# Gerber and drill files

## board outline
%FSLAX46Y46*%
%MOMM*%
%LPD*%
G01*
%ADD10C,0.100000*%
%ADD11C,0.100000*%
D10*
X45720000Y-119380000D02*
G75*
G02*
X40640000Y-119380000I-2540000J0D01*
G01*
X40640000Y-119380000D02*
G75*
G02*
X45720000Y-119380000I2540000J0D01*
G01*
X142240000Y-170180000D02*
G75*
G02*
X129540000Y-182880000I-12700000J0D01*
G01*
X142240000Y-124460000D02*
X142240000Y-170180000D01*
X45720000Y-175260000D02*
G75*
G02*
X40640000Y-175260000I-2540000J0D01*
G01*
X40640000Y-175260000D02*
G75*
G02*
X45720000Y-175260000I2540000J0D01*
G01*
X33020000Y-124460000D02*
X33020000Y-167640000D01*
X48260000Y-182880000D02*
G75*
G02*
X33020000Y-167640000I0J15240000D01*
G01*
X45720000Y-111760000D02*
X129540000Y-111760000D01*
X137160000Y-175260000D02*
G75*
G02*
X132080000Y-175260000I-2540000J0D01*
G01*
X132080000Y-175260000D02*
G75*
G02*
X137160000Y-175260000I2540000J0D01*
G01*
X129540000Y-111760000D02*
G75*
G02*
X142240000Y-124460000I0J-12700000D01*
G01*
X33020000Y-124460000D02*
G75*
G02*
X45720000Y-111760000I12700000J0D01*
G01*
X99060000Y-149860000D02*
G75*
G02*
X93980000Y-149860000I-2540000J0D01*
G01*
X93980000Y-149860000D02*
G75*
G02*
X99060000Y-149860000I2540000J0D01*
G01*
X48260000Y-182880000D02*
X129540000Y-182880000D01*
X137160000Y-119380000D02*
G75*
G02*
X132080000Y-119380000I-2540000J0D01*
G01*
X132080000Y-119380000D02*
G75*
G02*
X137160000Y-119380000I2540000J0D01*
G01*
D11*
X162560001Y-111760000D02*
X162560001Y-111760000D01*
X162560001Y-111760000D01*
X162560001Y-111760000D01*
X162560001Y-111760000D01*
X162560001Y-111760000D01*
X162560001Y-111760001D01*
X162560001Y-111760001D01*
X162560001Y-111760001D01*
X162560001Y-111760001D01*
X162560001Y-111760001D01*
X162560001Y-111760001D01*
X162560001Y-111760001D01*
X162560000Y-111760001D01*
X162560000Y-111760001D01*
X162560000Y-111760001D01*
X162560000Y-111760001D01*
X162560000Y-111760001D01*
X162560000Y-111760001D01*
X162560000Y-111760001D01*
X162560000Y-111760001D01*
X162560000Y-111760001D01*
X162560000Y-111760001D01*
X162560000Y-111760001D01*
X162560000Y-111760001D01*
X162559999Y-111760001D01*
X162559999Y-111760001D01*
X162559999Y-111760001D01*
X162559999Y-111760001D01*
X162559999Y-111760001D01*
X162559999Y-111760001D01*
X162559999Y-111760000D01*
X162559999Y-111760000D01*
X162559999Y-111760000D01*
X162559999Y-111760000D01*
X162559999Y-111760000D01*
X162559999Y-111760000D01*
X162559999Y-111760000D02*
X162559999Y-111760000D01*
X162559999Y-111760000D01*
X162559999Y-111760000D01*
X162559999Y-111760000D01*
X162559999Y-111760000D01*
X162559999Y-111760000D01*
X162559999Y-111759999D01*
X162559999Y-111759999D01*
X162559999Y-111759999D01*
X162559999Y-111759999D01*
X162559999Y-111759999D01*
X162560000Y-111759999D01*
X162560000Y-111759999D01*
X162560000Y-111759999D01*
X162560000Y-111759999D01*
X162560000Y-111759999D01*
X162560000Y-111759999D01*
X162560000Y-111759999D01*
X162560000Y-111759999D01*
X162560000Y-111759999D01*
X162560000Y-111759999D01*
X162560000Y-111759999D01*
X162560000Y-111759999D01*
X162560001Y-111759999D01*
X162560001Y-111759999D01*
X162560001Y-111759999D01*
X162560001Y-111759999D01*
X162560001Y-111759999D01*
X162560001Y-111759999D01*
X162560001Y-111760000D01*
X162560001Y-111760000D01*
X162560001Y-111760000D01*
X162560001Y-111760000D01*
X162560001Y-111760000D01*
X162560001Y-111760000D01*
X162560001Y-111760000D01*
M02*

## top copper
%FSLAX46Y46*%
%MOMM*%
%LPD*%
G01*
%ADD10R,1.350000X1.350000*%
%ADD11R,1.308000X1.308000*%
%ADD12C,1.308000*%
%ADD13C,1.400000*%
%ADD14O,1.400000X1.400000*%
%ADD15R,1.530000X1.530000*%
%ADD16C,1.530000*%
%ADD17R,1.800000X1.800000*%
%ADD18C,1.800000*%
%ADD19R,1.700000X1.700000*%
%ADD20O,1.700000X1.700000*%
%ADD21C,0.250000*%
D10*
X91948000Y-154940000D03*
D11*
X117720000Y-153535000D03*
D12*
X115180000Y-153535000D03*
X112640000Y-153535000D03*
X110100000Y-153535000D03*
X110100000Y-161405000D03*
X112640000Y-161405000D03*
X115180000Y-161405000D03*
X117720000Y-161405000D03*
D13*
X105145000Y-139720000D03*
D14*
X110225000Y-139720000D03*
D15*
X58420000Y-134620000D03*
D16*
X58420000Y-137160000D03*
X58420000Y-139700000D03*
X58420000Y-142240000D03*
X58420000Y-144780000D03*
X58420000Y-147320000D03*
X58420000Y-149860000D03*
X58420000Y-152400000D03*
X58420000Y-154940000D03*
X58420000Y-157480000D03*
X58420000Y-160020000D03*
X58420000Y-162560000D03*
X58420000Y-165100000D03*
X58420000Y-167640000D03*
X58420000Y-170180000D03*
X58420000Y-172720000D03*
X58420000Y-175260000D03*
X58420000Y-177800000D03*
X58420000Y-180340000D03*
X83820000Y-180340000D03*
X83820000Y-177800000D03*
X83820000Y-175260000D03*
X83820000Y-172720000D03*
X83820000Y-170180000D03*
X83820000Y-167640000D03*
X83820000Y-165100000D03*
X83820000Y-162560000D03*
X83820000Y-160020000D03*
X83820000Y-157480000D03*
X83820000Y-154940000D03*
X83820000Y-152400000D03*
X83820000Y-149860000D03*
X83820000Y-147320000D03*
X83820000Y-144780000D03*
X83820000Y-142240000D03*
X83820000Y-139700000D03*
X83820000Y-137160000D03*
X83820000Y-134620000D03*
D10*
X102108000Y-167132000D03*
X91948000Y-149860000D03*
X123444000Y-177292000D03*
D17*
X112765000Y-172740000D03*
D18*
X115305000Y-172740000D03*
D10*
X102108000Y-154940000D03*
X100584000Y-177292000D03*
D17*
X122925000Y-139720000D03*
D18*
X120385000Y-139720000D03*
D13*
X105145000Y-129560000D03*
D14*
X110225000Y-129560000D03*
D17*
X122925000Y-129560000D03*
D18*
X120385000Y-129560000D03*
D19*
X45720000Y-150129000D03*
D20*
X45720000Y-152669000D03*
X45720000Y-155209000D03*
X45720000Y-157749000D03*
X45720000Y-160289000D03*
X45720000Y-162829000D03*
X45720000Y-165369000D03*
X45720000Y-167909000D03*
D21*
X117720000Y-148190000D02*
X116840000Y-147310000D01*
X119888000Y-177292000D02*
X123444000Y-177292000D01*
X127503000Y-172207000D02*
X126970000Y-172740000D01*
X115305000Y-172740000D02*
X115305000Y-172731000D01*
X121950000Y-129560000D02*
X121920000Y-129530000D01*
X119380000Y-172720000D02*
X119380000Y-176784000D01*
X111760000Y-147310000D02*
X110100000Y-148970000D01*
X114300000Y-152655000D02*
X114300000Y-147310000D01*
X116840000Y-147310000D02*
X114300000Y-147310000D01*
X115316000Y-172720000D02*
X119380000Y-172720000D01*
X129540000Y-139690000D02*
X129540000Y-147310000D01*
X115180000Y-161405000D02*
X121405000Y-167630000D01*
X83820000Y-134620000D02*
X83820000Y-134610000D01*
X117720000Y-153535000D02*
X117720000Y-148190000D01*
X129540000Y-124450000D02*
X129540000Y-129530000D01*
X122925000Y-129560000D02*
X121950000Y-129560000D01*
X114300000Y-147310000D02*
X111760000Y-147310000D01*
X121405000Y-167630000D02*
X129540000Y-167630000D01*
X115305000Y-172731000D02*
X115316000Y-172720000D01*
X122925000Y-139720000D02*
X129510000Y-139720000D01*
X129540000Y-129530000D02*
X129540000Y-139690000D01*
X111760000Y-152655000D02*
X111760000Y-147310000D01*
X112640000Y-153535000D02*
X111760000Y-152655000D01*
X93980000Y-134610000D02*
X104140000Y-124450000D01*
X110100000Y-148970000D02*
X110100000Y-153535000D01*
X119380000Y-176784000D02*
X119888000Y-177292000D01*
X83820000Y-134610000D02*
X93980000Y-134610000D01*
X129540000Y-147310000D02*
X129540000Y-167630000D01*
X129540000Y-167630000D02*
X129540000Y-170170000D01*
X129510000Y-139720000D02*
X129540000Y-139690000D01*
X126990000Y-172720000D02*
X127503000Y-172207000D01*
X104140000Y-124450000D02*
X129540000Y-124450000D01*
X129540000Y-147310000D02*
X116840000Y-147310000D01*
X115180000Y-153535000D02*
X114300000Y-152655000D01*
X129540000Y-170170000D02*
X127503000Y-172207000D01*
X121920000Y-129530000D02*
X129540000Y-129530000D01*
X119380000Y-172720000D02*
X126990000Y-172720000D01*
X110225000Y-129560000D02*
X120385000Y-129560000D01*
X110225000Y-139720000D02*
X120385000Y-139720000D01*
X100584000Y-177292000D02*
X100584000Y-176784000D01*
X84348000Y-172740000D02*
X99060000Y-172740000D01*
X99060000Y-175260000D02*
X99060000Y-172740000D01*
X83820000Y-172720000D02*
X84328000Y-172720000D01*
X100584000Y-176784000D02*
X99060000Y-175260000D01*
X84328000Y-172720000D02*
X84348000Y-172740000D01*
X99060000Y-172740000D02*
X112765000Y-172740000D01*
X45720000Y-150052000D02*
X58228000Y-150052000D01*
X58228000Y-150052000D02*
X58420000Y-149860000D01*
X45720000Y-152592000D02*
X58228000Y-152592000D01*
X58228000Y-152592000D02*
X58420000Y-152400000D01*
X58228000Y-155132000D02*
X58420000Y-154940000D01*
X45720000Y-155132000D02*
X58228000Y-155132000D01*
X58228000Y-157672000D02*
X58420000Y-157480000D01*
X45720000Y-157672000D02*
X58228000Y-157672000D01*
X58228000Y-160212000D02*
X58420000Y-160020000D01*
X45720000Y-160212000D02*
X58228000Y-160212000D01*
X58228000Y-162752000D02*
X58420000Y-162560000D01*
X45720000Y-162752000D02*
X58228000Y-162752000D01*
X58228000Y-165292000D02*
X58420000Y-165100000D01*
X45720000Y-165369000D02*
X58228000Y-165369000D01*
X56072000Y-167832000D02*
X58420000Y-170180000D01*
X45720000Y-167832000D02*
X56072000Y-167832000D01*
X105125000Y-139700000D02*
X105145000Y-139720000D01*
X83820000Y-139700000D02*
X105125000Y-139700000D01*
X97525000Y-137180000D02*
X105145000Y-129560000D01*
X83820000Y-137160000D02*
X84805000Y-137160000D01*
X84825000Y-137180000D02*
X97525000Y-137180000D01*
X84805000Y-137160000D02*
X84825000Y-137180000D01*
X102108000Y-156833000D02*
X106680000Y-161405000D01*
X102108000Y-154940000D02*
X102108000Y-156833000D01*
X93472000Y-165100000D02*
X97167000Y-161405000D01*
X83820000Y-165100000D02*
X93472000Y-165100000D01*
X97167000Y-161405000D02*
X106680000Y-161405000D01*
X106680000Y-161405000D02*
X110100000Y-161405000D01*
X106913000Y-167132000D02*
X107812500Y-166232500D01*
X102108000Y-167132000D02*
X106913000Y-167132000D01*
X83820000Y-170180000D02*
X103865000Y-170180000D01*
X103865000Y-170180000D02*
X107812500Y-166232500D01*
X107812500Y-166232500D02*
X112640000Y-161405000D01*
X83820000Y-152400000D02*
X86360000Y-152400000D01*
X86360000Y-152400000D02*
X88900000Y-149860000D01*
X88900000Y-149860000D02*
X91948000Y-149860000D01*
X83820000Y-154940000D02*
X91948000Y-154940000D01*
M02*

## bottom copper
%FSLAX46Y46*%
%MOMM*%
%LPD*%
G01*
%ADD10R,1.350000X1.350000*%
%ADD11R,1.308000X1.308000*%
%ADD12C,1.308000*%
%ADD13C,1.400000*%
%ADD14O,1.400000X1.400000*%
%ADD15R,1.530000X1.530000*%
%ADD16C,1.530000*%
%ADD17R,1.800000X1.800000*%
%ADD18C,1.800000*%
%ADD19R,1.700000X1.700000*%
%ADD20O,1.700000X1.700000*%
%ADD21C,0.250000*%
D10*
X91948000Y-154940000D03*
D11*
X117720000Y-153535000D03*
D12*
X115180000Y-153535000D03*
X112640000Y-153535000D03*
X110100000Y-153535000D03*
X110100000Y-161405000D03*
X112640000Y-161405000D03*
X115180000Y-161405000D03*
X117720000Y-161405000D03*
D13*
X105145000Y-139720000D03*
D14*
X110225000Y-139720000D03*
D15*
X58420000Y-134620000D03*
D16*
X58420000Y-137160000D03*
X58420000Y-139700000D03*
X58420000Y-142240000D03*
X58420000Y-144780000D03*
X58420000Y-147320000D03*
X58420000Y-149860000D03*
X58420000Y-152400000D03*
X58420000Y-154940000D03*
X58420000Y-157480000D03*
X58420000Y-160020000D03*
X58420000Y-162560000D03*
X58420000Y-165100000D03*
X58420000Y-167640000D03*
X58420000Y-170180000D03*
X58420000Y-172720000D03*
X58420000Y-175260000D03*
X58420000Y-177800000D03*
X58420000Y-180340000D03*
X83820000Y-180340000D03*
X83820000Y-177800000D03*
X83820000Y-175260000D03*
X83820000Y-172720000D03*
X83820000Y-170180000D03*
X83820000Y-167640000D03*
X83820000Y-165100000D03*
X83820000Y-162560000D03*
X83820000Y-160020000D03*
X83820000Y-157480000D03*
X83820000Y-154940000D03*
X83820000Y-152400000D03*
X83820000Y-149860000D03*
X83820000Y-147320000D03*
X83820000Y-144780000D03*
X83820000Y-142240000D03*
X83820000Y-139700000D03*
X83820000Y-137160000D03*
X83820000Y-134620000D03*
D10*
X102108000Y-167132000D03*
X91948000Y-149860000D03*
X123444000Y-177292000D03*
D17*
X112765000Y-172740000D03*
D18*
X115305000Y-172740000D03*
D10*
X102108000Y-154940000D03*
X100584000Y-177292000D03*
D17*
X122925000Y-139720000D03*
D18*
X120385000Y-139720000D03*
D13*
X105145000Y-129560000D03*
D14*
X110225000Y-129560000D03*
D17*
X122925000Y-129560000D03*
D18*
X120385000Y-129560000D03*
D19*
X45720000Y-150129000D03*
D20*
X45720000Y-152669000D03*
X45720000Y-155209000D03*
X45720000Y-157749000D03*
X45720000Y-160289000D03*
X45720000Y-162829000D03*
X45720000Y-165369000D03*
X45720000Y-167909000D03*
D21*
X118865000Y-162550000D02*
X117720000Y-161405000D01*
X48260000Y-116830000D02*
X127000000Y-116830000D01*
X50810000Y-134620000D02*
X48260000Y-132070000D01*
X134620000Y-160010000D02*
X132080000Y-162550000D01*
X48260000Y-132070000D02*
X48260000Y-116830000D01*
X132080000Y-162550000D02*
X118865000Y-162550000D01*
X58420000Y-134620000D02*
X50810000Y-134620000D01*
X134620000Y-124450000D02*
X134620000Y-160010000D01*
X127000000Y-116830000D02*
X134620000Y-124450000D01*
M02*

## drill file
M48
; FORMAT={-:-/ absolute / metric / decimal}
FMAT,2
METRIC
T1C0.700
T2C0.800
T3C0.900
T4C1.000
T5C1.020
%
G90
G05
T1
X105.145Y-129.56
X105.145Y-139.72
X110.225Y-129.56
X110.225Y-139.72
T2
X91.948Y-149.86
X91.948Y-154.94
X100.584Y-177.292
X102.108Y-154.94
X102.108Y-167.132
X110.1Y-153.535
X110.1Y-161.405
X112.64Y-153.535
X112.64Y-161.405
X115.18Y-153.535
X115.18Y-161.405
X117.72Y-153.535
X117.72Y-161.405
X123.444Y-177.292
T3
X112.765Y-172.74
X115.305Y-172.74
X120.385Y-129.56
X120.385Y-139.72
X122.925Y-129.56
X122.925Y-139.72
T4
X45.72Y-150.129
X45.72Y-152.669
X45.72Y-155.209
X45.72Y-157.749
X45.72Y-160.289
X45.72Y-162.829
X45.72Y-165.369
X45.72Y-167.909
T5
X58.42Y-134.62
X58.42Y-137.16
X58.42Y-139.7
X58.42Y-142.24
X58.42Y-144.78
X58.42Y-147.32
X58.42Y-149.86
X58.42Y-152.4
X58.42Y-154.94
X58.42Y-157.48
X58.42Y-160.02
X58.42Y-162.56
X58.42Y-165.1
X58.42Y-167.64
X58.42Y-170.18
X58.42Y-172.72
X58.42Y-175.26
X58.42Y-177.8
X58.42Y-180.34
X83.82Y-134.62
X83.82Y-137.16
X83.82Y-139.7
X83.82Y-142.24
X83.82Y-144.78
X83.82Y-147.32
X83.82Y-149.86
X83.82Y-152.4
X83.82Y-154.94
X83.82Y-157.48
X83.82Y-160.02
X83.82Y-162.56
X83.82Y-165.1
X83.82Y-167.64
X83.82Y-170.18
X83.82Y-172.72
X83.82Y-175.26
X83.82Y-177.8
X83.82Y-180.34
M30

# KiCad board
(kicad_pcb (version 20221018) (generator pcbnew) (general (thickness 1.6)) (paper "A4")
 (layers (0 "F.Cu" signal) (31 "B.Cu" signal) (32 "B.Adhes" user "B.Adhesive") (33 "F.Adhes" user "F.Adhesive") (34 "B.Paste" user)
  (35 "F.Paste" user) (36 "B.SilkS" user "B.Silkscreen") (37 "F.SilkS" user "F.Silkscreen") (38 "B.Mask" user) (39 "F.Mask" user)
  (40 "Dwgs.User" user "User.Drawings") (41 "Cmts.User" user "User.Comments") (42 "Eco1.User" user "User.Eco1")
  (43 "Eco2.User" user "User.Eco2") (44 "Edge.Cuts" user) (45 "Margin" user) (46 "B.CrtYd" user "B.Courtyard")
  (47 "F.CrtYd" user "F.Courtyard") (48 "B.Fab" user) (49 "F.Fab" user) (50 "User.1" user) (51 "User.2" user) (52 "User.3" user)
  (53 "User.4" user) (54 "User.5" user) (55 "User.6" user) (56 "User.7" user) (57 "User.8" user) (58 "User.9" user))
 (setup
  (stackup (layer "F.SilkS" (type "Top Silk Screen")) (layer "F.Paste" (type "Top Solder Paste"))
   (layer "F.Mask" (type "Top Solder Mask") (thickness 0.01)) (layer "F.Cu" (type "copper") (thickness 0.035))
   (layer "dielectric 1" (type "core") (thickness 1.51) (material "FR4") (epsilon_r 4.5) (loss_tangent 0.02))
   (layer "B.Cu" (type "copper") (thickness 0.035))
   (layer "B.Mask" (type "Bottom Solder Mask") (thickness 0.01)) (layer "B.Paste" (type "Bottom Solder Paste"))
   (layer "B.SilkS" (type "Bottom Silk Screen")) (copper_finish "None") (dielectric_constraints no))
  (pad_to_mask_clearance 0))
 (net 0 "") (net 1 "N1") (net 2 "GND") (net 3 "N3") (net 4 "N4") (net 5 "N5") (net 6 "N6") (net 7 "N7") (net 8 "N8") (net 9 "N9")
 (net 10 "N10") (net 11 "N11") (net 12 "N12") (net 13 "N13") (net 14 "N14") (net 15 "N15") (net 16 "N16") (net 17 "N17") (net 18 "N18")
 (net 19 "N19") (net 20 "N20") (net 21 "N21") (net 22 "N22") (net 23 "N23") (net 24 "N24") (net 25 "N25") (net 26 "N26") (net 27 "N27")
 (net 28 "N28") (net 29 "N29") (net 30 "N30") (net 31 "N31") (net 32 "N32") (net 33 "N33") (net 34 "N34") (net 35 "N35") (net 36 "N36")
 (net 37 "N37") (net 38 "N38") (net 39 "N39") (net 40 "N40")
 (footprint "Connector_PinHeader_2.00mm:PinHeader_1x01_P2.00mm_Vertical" (layer "F.Cu") (at 91.948 154.94)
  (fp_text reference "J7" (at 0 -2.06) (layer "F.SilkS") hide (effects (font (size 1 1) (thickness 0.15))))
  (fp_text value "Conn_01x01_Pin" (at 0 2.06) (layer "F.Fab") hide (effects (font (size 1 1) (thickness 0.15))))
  (pad "1" thru_hole rect (at 0 0) (size 1.35 1.35) (drill 0.8) (layers "*.Cu" "*.Mask") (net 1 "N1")))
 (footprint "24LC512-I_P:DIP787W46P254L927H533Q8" (layer "F.Cu") (at 113.91 157.47 -90)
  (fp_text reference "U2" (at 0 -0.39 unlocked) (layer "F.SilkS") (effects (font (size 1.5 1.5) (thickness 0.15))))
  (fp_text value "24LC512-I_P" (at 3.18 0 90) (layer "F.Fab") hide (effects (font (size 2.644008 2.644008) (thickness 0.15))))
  (pad "1" thru_hole rect (at -3.935 -3.81 270) (size 1.308 1.308) (drill 0.8) (layers "*.Cu" "*.Mask") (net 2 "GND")
   (solder_mask_margin 0.102))
  (pad "2" thru_hole circle (at -3.935 -1.27 270) (size 1.308 1.308) (drill 0.8) (layers "*.Cu" "*.Mask") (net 2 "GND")
   (solder_mask_margin 0.102))
  (pad "3" thru_hole circle (at -3.935 1.27 270) (size 1.308 1.308) (drill 0.8) (layers "*.Cu" "*.Mask") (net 2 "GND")
   (solder_mask_margin 0.102))
  (pad "4" thru_hole circle (at -3.935 3.81 270) (size 1.308 1.308) (drill 0.8) (layers "*.Cu" "*.Mask") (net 2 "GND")
   (solder_mask_margin 0.102))
  (pad "5" thru_hole circle (at 3.935 3.81 270) (size 1.308 1.308) (drill 0.8) (layers "*.Cu" "*.Mask") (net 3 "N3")
   (solder_mask_margin 0.102))
  (pad "6" thru_hole circle (at 3.935 1.27 270) (size 1.308 1.308) (drill 0.8) (layers "*.Cu" "*.Mask") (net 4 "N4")
   (solder_mask_margin 0.102))
  (pad "7" thru_hole circle (at 3.935 -1.27 270) (size 1.308 1.308) (drill 0.8) (layers "*.Cu" "*.Mask") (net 2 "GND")
   (solder_mask_margin 0.102))
  (pad "8" thru_hole circle (at 3.935 -3.81 270) (size 1.308 1.308) (drill 0.8) (layers "*.Cu" "*.Mask") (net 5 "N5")
   (solder_mask_margin 0.102)))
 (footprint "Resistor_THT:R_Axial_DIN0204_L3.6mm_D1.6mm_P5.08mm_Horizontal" (layer "F.Cu") (at 105.145 139.72)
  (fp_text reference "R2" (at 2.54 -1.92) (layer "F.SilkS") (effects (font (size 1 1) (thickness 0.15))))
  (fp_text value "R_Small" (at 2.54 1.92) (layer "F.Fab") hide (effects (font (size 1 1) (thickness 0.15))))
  (pad "1" thru_hole circle (at 0 0) (size 1.4 1.4) (drill 0.7) (layers "*.Cu" "*.Mask") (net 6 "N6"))
  (pad "2" thru_hole oval (at 5.08 0) (size 1.4 1.4) (drill 0.7) (layers "*.Cu" "*.Mask") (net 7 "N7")))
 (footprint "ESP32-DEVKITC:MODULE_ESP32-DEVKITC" (layer "F.Cu") (at 71.12 157.47)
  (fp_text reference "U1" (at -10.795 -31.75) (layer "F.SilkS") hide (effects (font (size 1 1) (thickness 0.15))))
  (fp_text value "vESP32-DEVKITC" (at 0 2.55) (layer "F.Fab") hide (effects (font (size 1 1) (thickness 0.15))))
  (pad "1" thru_hole rect (at -12.7 -22.85) (size 1.53 1.53) (drill 1.02) (layers "*.Cu" "*.Mask") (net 5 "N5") (solder_mask_margin 0.102))
  (pad "2" thru_hole circle (at -12.7 -20.31) (size 1.53 1.53) (drill 1.02) (layers "*.Cu" "*.Mask") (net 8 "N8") (solder_mask_margin 0.102))
  (pad "3" thru_hole circle (at -12.7 -17.77) (size 1.53 1.53) (drill 1.02) (layers "*.Cu" "*.Mask") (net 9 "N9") (solder_mask_margin 0.102))
  (pad "4" thru_hole circle (at -12.7 -15.23) (size 1.53 1.53) (drill 1.02) (layers "*.Cu" "*.Mask") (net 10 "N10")
   (solder_mask_margin 0.102))
  (pad "5" thru_hole circle (at -12.7 -12.69) (size 1.53 1.53) (drill 1.02) (layers "*.Cu" "*.Mask") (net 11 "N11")
   (solder_mask_margin 0.102))
  (pad "6" thru_hole circle (at -12.7 -10.15) (size 1.53 1.53) (drill 1.02) (layers "*.Cu" "*.Mask") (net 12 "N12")
   (solder_mask_margin 0.102))
  (pad "7" thru_hole circle (at -12.7 -7.61) (size 1.53 1.53) (drill 1.02) (layers "*.Cu" "*.Mask") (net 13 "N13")
   (solder_mask_margin 0.102))
  (pad "8" thru_hole circle (at -12.7 -5.07) (size 1.53 1.53) (drill 1.02) (layers "*.Cu" "*.Mask") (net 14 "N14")
   (solder_mask_margin 0.102))
  (pad "9" thru_hole circle (at -12.7 -2.53) (size 1.53 1.53) (drill 1.02) (layers "*.Cu" "*.Mask") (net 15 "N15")
   (solder_mask_margin 0.102))
  (pad "10" thru_hole circle (at -12.7 0.01) (size 1.53 1.53) (drill 1.02) (layers "*.Cu" "*.Mask") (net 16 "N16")
   (solder_mask_margin 0.102))
  (pad "11" thru_hole circle (at -12.7 2.55) (size 1.53 1.53) (drill 1.02) (layers "*.Cu" "*.Mask") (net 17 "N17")
   (solder_mask_margin 0.102))
  (pad "12" thru_hole circle (at -12.7 5.09) (size 1.53 1.53) (drill 1.02) (layers "*.Cu" "*.Mask") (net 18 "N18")
   (solder_mask_margin 0.102))
  (pad "13" thru_hole circle (at -12.7 7.63) (size 1.53 1.53) (drill 1.02) (layers "*.Cu" "*.Mask") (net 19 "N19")
   (solder_mask_margin 0.102))
  (pad "14" thru_hole circle (at -12.7 10.17) (size 1.53 1.53) (drill 1.02) (layers "*.Cu" "*.Mask") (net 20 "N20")
   (solder_mask_margin 0.102))
  (pad "15" thru_hole circle (at -12.7 12.71) (size 1.53 1.53) (drill 1.02) (layers "*.Cu" "*.Mask") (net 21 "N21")
   (solder_mask_margin 0.102))
  (pad "16" thru_hole circle (at -12.7 15.25) (size 1.53 1.53) (drill 1.02) (layers "*.Cu" "*.Mask") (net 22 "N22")
   (solder_mask_margin 0.102))
  (pad "17" thru_hole circle (at -12.7 17.79) (size 1.53 1.53) (drill 1.02) (layers "*.Cu" "*.Mask") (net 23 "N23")
   (solder_mask_margin 0.102))
  (pad "18" thru_hole circle (at -12.7 20.33) (size 1.53 1.53) (drill 1.02) (layers "*.Cu" "*.Mask") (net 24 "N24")
   (solder_mask_margin 0.102))
  (pad "19" thru_hole circle (at -12.7 22.87) (size 1.53 1.53) (drill 1.02) (layers "*.Cu" "*.Mask") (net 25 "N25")
   (solder_mask_margin 0.102))
  (pad "20" thru_hole circle (at 12.7 22.87) (size 1.53 1.53) (drill 1.02) (layers "*.Cu" "*.Mask") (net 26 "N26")
   (solder_mask_margin 0.102))
  (pad "21" thru_hole circle (at 12.7 20.33) (size 1.53 1.53) (drill 1.02) (layers "*.Cu" "*.Mask") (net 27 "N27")
   (solder_mask_margin 0.102))
  (pad "22" thru_hole circle (at 12.7 17.79) (size 1.53 1.53) (drill 1.02) (layers "*.Cu" "*.Mask") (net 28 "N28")
   (solder_mask_margin 0.102))
  (pad "23" thru_hole circle (at 12.7 15.25) (size 1.53 1.53) (drill 1.02) (layers "*.Cu" "*.Mask") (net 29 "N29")
   (solder_mask_margin 0.102))
  (pad "24" thru_hole circle (at 12.7 12.71) (size 1.53 1.53) (drill 1.02) (layers "*.Cu" "*.Mask") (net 4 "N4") (solder_mask_margin 0.102))
  (pad "25" thru_hole circle (at 12.7 10.17) (size 1.53 1.53) (drill 1.02) (layers "*.Cu" "*.Mask") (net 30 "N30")
   (solder_mask_margin 0.102))
  (pad "26" thru_hole circle (at 12.7 7.63) (size 1.53 1.53) (drill 1.02) (layers "*.Cu" "*.Mask") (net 3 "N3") (solder_mask_margin 0.102))
  (pad "27" thru_hole circle (at 12.7 5.09) (size 1.53 1.53) (drill 1.02) (layers "*.Cu" "*.Mask") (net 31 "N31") (solder_mask_margin 0.102))
  (pad "28" thru_hole circle (at 12.7 2.55) (size 1.53 1.53) (drill 1.02) (layers "*.Cu" "*.Mask") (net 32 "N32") (solder_mask_margin 0.102))
  (pad "29" thru_hole circle (at 12.7 0.01) (size 1.53 1.53) (drill 1.02) (layers "*.Cu" "*.Mask") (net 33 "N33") (solder_mask_margin 0.102))
  (pad "30" thru_hole circle (at 12.7 -2.53) (size 1.53 1.53) (drill 1.02) (layers "*.Cu" "*.Mask") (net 1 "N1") (solder_mask_margin 0.102))
  (pad "31" thru_hole circle (at 12.7 -5.07) (size 1.53 1.53) (drill 1.02) (layers "*.Cu" "*.Mask") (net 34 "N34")
   (solder_mask_margin 0.102))
  (pad "32" thru_hole circle (at 12.7 -7.61) (size 1.53 1.53) (drill 1.02) (layers "*.Cu" "*.Mask") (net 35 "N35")
   (solder_mask_margin 0.102))
  (pad "33" thru_hole circle (at 12.7 -10.15) (size 1.53 1.53) (drill 1.02) (layers "*.Cu" "*.Mask") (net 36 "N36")
   (solder_mask_margin 0.102))
  (pad "34" thru_hole circle (at 12.7 -12.69) (size 1.53 1.53) (drill 1.02) (layers "*.Cu" "*.Mask") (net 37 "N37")
   (solder_mask_margin 0.102))
  (pad "35" thru_hole circle (at 12.7 -15.23) (size 1.53 1.53) (drill 1.02) (layers "*.Cu" "*.Mask") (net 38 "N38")
   (solder_mask_margin 0.102))
  (pad "36" thru_hole circle (at 12.7 -17.77) (size 1.53 1.53) (drill 1.02) (layers "*.Cu" "*.Mask") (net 6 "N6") (solder_mask_margin 0.102))
  (pad "37" thru_hole circle (at 12.7 -20.31) (size 1.53 1.53) (drill 1.02) (layers "*.Cu" "*.Mask") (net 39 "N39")
   (solder_mask_margin 0.102))
  (pad "38" thru_hole circle (at 12.7 -22.85) (size 1.53 1.53) (drill 1.02) (layers "*.Cu" "*.Mask") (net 2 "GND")
   (solder_mask_margin 0.102)))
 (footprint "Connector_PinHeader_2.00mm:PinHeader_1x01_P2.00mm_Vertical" (layer "F.Cu") (at 102.108 167.132)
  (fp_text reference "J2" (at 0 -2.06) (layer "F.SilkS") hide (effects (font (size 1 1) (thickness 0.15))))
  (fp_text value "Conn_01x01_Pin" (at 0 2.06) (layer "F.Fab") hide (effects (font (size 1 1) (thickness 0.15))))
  (pad "1" thru_hole rect (at 0 0) (size 1.35 1.35) (drill 0.8) (layers "*.Cu" "*.Mask") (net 4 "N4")))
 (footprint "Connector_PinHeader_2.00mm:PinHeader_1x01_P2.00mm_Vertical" (layer "F.Cu") (at 91.948 149.86)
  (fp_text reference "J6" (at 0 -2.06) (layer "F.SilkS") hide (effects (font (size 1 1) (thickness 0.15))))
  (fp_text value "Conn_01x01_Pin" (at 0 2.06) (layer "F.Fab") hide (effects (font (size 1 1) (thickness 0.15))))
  (pad "1" thru_hole rect (at 0 0) (size 1.35 1.35) (drill 0.8) (layers "*.Cu" "*.Mask") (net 34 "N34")))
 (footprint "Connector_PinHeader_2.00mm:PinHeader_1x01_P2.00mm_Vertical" (layer "F.Cu") (at 123.444 177.292)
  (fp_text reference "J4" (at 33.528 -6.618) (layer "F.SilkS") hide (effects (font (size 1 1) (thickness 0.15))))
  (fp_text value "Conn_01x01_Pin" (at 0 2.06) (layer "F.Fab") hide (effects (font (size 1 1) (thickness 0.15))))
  (pad "1" thru_hole rect (at 0 0) (size 1.35 1.35) (drill 0.8) (layers "*.Cu" "*.Mask") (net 2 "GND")))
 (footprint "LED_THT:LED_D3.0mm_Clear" (layer "F.Cu") (at 112.765 172.74)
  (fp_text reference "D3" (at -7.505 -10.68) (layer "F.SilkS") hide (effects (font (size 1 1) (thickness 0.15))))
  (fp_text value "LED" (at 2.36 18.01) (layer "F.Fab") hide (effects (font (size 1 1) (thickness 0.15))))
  (pad "1" thru_hole rect (at 0 0) (size 1.8 1.8) (drill 0.9) (layers "*.Cu" "*.Mask") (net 29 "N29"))
  (pad "2" thru_hole circle (at 2.54 0) (size 1.8 1.8) (drill 0.9) (layers "*.Cu" "*.Mask") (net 2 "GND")))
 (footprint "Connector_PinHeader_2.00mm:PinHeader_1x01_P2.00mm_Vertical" (layer "F.Cu") (at 102.108 154.94)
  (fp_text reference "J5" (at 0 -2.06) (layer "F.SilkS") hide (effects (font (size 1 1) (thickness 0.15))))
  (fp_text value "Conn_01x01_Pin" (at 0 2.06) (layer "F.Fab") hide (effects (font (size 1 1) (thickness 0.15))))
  (pad "1" thru_hole rect (at 0 0) (size 1.35 1.35) (drill 0.8) (layers "*.Cu" "*.Mask") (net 3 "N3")))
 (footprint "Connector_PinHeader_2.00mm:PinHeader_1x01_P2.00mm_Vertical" (layer "F.Cu") (at 100.584 177.292)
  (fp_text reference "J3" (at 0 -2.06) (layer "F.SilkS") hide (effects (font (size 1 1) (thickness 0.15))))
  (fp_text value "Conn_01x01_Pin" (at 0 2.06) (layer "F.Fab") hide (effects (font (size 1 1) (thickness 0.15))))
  (pad "1" thru_hole rect (at 0 0) (size 1.35 1.35) (drill 0.8) (layers "*.Cu" "*.Mask") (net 29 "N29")))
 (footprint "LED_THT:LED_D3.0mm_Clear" (layer "F.Cu") (at 122.925 139.72 180)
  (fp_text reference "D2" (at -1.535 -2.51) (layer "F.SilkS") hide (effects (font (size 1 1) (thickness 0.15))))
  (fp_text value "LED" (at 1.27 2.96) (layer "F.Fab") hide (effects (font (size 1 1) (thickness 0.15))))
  (pad "1" thru_hole rect (at 0 0 180) (size 1.8 1.8) (drill 0.9) (layers "*.Cu" "*.Mask") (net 2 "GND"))
  (pad "2" thru_hole circle (at 2.54 0 180) (size 1.8 1.8) (drill 0.9) (layers "*.Cu" "*.Mask") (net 7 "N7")))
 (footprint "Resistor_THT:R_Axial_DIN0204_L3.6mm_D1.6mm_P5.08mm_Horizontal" (layer "F.Cu") (at 105.145 129.56)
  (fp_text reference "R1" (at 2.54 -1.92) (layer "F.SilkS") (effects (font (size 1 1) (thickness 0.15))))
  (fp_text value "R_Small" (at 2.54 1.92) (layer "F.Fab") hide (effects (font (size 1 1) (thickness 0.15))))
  (pad "1" thru_hole circle (at 0 0) (size 1.4 1.4) (drill 0.7) (layers "*.Cu" "*.Mask") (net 39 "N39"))
  (pad "2" thru_hole oval (at 5.08 0) (size 1.4 1.4) (drill 0.7) (layers "*.Cu" "*.Mask") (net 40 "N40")))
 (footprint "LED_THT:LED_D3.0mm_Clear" (layer "F.Cu") (at 122.925 129.56 180)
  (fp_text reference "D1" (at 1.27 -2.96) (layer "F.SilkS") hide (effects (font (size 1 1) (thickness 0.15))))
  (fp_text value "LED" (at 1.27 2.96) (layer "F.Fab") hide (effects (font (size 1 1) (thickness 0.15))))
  (pad "1" thru_hole rect (at 0 0 180) (size 1.8 1.8) (drill 0.9) (layers "*.Cu" "*.Mask") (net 2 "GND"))
  (pad "2" thru_hole circle (at 2.54 0 180) (size 1.8 1.8) (drill 0.9) (layers "*.Cu" "*.Mask") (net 40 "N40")))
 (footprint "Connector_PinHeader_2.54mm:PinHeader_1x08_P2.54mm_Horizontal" (layer "B.Cu") (at 45.72 150.129 180)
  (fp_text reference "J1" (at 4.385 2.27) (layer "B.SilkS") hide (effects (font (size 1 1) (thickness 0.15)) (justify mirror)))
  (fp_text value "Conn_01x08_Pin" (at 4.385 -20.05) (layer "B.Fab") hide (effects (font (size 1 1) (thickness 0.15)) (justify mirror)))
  (pad "1" thru_hole rect (at 0 0 180) (size 1.7 1.7) (drill 1) (layers "*.Cu" "*.Mask") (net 13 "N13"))
  (pad "2" thru_hole oval (at 0 -2.54 180) (size 1.7 1.7) (drill 1) (layers "*.Cu" "*.Mask") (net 14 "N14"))
  (pad "3" thru_hole oval (at 0 -5.08 180) (size 1.7 1.7) (drill 1) (layers "*.Cu" "*.Mask") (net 15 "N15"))
  (pad "4" thru_hole oval (at 0 -7.62 180) (size 1.7 1.7) (drill 1) (layers "*.Cu" "*.Mask") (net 16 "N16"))
  (pad "5" thru_hole oval (at 0 -10.16 180) (size 1.7 1.7) (drill 1) (layers "*.Cu" "*.Mask") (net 17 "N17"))
  (pad "6" thru_hole oval (at 0 -12.7 180) (size 1.7 1.7) (drill 1) (layers "*.Cu" "*.Mask") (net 18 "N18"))
  (pad "7" thru_hole oval (at 0 -15.24 180) (size 1.7 1.7) (drill 1) (layers "*.Cu" "*.Mask") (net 19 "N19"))
  (pad "8" thru_hole oval (at 0 -17.78 180) (size 1.7 1.7) (drill 1) (layers "*.Cu" "*.Mask") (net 21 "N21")))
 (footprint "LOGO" (layer "B.Cu") (at 68.520868 155.367556 180)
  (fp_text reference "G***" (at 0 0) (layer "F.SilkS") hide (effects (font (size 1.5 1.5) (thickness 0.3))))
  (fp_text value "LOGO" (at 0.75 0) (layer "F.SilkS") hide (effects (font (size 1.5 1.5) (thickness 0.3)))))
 (gr_circle (center 43.18 119.38) (end 43.18 116.84) (stroke (width 0.1) (type default)) (fill none) (layer "Edge.Cuts"))
 (gr_arc (start 142.24 170.18) (mid 138.520256 179.160256) (end 129.54 182.88) (stroke (width 0.1) (type default)) (layer "Edge.Cuts"))
 (gr_line (start 142.24 124.46) (end 142.24 170.18) (stroke (width 0.1) (type default)) (layer "Edge.Cuts"))
 (gr_circle (center 43.18 175.26) (end 43.18 172.72) (stroke (width 0.1) (type default)) (fill none) (layer "Edge.Cuts"))
 (gr_line (start 33.02 124.46) (end 33.02 167.64) (stroke (width 0.1) (type default)) (layer "Edge.Cuts"))
 (gr_arc (start 48.26 182.88) (mid 37.483693 178.416307) (end 33.02 167.64) (stroke (width 0.1) (type default)) (layer "Edge.Cuts"))
 (gr_line (start 45.72 111.76) (end 129.54 111.76) (stroke (width 0.1) (type default)) (layer "Edge.Cuts"))
 (gr_circle (center 134.62 175.26) (end 134.62 172.72) (stroke (width 0.1) (type default)) (fill none) (layer "Edge.Cuts"))
 (gr_arc (start 129.54 111.76) (mid 138.520256 115.479744) (end 142.24 124.46) (stroke (width 0.1) (type default)) (layer "Edge.Cuts"))
 (gr_arc (start 33.02 124.46) (mid 36.739744 115.479744) (end 45.72 111.76) (stroke (width 0.1) (type default)) (layer "Edge.Cuts"))
 (gr_circle (center 96.52 149.86) (end 96.52 147.32) (stroke (width 0.1) (type default)) (fill none) (layer "Edge.Cuts"))
 (gr_line (start 48.26 182.88) (end 129.54 182.88) (stroke (width 0.1) (type default)) (layer "Edge.Cuts"))
 (gr_circle (center 134.62 119.38) (end 134.62 116.84) (stroke (width 0.1) (type default)) (fill none) (layer "Edge.Cuts"))
 (gr_circle (center 162.56 111.76) (end 162.56 111.76) (stroke (width 0.1) (type default)) (fill none) (layer "Edge.Cuts"))
 (segment (start 117.72 148.19) (end 116.84 147.31) (width 0.25) (layer "F.Cu") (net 2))
 (segment (start 119.888 177.292) (end 123.444 177.292) (width 0.25) (layer "F.Cu") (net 2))
 (segment (start 127.503 172.207) (end 126.97 172.74) (width 0.25) (layer "F.Cu") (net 2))
 (segment (start 115.305 172.74) (end 115.305 172.731) (width 0.25) (layer "F.Cu") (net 2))
 (segment (start 121.95 129.56) (end 121.92 129.53) (width 0.25) (layer "F.Cu") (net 2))
 (segment (start 119.38 172.72) (end 119.38 176.784) (width 0.25) (layer "F.Cu") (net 2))
 (segment (start 111.76 147.31) (end 110.1 148.97) (width 0.25) (layer "F.Cu") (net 2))
 (segment (start 114.3 152.655) (end 114.3 147.31) (width 0.25) (layer "F.Cu") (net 2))
 (segment (start 116.84 147.31) (end 114.3 147.31) (width 0.25) (layer "F.Cu") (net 2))
 (segment (start 115.316 172.72) (end 119.38 172.72) (width 0.25) (layer "F.Cu") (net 2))
 (segment (start 129.54 139.69) (end 129.54 147.31) (width 0.25) (layer "F.Cu") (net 2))
 (segment (start 115.18 161.405) (end 121.405 167.63) (width 0.25) (layer "F.Cu") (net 2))
 (segment (start 83.82 134.62) (end 83.82 134.61) (width 0.25) (layer "F.Cu") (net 2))
 (segment (start 117.72 153.535) (end 117.72 148.19) (width 0.25) (layer "F.Cu") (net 2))
 (segment (start 129.54 124.45) (end 129.54 129.53) (width 0.25) (layer "F.Cu") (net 2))
 (segment (start 122.925 129.56) (end 121.95 129.56) (width 0.25) (layer "F.Cu") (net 2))
 (segment (start 114.3 147.31) (end 111.76 147.31) (width 0.25) (layer "F.Cu") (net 2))
 (segment (start 121.405 167.63) (end 129.54 167.63) (width 0.25) (layer "F.Cu") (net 2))
 (segment (start 115.305 172.731) (end 115.316 172.72) (width 0.25) (layer "F.Cu") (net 2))
 (segment (start 122.925 139.72) (end 129.51 139.72) (width 0.25) (layer "F.Cu") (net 2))
 (segment (start 129.54 129.53) (end 129.54 139.69) (width 0.25) (layer "F.Cu") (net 2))
 (segment (start 111.76 152.655) (end 111.76 147.31) (width 0.25) (layer "F.Cu") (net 2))
 (segment (start 112.64 153.535) (end 111.76 152.655) (width 0.25) (layer "F.Cu") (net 2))
 (segment (start 93.98 134.61) (end 104.14 124.45) (width 0.25) (layer "F.Cu") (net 2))
 (segment (start 110.1 148.97) (end 110.1 153.535) (width 0.25) (layer "F.Cu") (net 2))
 (segment (start 119.38 176.784) (end 119.888 177.292) (width 0.25) (layer "F.Cu") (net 2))
 (segment (start 83.82 134.61) (end 93.98 134.61) (width 0.25) (layer "F.Cu") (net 2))
 (segment (start 129.54 147.31) (end 129.54 167.63) (width 0.25) (layer "F.Cu") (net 2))
 (segment (start 129.54 167.63) (end 129.54 170.17) (width 0.25) (layer "F.Cu") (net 2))
 (segment (start 129.51 139.72) (end 129.54 139.69) (width 0.25) (layer "F.Cu") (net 2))
 (segment (start 126.99 172.72) (end 127.503 172.207) (width 0.25) (layer "F.Cu") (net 2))
 (segment (start 104.14 124.45) (end 129.54 124.45) (width 0.25) (layer "F.Cu") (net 2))
 (segment (start 129.54 147.31) (end 116.84 147.31) (width 0.25) (layer "F.Cu") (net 2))
 (segment (start 115.18 153.535) (end 114.3 152.655) (width 0.25) (layer "F.Cu") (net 2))
 (segment (start 129.54 170.17) (end 127.503 172.207) (width 0.25) (layer "F.Cu") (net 2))
 (segment (start 121.92 129.53) (end 129.54 129.53) (width 0.25) (layer "F.Cu") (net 2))
 (segment (start 119.38 172.72) (end 126.99 172.72) (width 0.25) (layer "F.Cu") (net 2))
 (segment (start 110.225 129.56) (end 120.385 129.56) (width 0.25) (layer "F.Cu") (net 40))
 (segment (start 110.225 139.72) (end 120.385 139.72) (width 0.25) (layer "F.Cu") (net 7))
 (segment (start 100.584 177.292) (end 100.584 176.784) (width 0.25) (layer "F.Cu") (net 29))
 (segment (start 84.348 172.74) (end 99.06 172.74) (width 0.25) (layer "F.Cu") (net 29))
 (segment (start 99.06 175.26) (end 99.06 172.74) (width 0.25) (layer "F.Cu") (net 29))
 (segment (start 83.82 172.72) (end 84.328 172.72) (width 0.25) (layer "F.Cu") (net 29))
 (segment (start 100.584 176.784) (end 99.06 175.26) (width 0.25) (layer "F.Cu") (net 29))
 (segment (start 84.328 172.72) (end 84.348 172.74) (width 0.25) (layer "F.Cu") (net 29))
 (segment (start 99.06 172.74) (end 112.765 172.74) (width 0.25) (layer "F.Cu") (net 29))
 (segment (start 45.72 150.052) (end 58.228 150.052) (width 0.25) (layer "F.Cu") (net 13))
 (segment (start 58.228 150.052) (end 58.42 149.86) (width 0.25) (layer "F.Cu") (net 13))
 (segment (start 45.72 152.592) (end 58.228 152.592) (width 0.25) (layer "F.Cu") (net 14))
 (segment (start 58.228 152.592) (end 58.42 152.4) (width 0.25) (layer "F.Cu") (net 14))
 (segment (start 58.228 155.132) (end 58.42 154.94) (width 0.25) (layer "F.Cu") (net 15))
 (segment (start 45.72 155.132) (end 58.228 155.132) (width 0.25) (layer "F.Cu") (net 15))
 (segment (start 58.228 157.672) (end 58.42 157.48) (width 0.25) (layer "F.Cu") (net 16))
 (segment (start 45.72 157.672) (end 58.228 157.672) (width 0.25) (layer "F.Cu") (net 16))
 (segment (start 58.228 160.212) (end 58.42 160.02) (width 0.25) (layer "F.Cu") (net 17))
 (segment (start 45.72 160.212) (end 58.228 160.212) (width 0.25) (layer "F.Cu") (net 17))
 (segment (start 58.228 162.752) (end 58.42 162.56) (width 0.25) (layer "F.Cu") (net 18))
 (segment (start 45.72 162.752) (end 58.228 162.752) (width 0.25) (layer "F.Cu") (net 18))
 (segment (start 58.228 165.292) (end 58.42 165.1) (width 0.25) (layer "F.Cu") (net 19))
 (segment (start 45.72 165.369) (end 58.228 165.369) (width 0.25) (layer "F.Cu") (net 19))
 (segment (start 56.072 167.832) (end 58.42 170.18) (width 0.25) (layer "F.Cu") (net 21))
 (segment (start 45.72 167.832) (end 56.072 167.832) (width 0.25) (layer "F.Cu") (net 21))
 (segment (start 105.125 139.7) (end 105.145 139.72) (width 0.25) (layer "F.Cu") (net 6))
 (segment (start 83.82 139.7) (end 105.125 139.7) (width 0.25) (layer "F.Cu") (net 6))
 (segment (start 97.525 137.18) (end 105.145 129.56) (width 0.25) (layer "F.Cu") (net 39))
 (segment (start 83.82 137.16) (end 84.805 137.16) (width 0.25) (layer "F.Cu") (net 39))
 (segment (start 84.825 137.18) (end 97.525 137.18) (width 0.25) (layer "F.Cu") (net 39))
 (segment (start 84.805 137.16) (end 84.825 137.18) (width 0.25) (layer "F.Cu") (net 39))
 (segment (start 118.865 162.55) (end 117.72 161.405) (width 0.25) (layer "B.Cu") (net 5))
 (segment (start 48.26 116.83) (end 127 116.83) (width 0.25) (layer "B.Cu") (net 5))
 (segment (start 50.81 134.62) (end 48.26 132.07) (width 0.25) (layer "B.Cu") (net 5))
 (segment (start 134.62 160.01) (end 132.08 162.55) (width 0.25) (layer "B.Cu") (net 5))
 (segment (start 48.26 132.07) (end 48.26 116.83) (width 0.25) (layer "B.Cu") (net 5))
 (segment (start 132.08 162.55) (end 118.865 162.55) (width 0.25) (layer "B.Cu") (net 5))
 (segment (start 58.42 134.62) (end 50.81 134.62) (width 0.25) (layer "B.Cu") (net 5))
 (segment (start 134.62 124.45) (end 134.62 160.01) (width 0.25) (layer "B.Cu") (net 5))
 (segment (start 127 116.83) (end 134.62 124.45) (width 0.25) (layer "B.Cu") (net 5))
 (segment (start 102.108 156.833) (end 106.68 161.405) (width 0.25) (layer "F.Cu") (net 3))
 (segment (start 102.108 154.94) (end 102.108 156.833) (width 0.25) (layer "F.Cu") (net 3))
 (segment (start 93.472 165.1) (end 97.167 161.405) (width 0.25) (layer "F.Cu") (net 3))
 (segment (start 83.82 165.1) (end 93.472 165.1) (width 0.25) (layer "F.Cu") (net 3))
 (segment (start 97.167 161.405) (end 106.68 161.405) (width 0.25) (layer "F.Cu") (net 3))
 (segment (start 106.68 161.405) (end 110.1 161.405) (width 0.25) (layer "F.Cu") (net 3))
 (segment (start 106.913 167.132) (end 107.8125 166.2325) (width 0.25) (layer "F.Cu") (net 4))
 (segment (start 102.108 167.132) (end 106.913 167.132) (width 0.25) (layer "F.Cu") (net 4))
 (segment (start 83.82 170.18) (end 103.865 170.18) (width 0.25) (layer "F.Cu") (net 4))
 (segment (start 103.865 170.18) (end 107.8125 166.2325) (width 0.25) (layer "F.Cu") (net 4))
 (segment (start 107.8125 166.2325) (end 112.64 161.405) (width 0.25) (layer "F.Cu") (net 4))
 (segment (start 83.82 152.4) (end 86.36 152.4) (width 0.25) (layer "F.Cu") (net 34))
 (segment (start 86.36 152.4) (end 88.9 149.86) (width 0.25) (layer "F.Cu") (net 34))
 (segment (start 88.9 149.86) (end 91.948 149.86) (width 0.25) (layer "F.Cu") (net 34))
 (segment (start 83.82 154.94) (end 91.948 154.94) (width 0.25) (layer "F.Cu") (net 1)))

